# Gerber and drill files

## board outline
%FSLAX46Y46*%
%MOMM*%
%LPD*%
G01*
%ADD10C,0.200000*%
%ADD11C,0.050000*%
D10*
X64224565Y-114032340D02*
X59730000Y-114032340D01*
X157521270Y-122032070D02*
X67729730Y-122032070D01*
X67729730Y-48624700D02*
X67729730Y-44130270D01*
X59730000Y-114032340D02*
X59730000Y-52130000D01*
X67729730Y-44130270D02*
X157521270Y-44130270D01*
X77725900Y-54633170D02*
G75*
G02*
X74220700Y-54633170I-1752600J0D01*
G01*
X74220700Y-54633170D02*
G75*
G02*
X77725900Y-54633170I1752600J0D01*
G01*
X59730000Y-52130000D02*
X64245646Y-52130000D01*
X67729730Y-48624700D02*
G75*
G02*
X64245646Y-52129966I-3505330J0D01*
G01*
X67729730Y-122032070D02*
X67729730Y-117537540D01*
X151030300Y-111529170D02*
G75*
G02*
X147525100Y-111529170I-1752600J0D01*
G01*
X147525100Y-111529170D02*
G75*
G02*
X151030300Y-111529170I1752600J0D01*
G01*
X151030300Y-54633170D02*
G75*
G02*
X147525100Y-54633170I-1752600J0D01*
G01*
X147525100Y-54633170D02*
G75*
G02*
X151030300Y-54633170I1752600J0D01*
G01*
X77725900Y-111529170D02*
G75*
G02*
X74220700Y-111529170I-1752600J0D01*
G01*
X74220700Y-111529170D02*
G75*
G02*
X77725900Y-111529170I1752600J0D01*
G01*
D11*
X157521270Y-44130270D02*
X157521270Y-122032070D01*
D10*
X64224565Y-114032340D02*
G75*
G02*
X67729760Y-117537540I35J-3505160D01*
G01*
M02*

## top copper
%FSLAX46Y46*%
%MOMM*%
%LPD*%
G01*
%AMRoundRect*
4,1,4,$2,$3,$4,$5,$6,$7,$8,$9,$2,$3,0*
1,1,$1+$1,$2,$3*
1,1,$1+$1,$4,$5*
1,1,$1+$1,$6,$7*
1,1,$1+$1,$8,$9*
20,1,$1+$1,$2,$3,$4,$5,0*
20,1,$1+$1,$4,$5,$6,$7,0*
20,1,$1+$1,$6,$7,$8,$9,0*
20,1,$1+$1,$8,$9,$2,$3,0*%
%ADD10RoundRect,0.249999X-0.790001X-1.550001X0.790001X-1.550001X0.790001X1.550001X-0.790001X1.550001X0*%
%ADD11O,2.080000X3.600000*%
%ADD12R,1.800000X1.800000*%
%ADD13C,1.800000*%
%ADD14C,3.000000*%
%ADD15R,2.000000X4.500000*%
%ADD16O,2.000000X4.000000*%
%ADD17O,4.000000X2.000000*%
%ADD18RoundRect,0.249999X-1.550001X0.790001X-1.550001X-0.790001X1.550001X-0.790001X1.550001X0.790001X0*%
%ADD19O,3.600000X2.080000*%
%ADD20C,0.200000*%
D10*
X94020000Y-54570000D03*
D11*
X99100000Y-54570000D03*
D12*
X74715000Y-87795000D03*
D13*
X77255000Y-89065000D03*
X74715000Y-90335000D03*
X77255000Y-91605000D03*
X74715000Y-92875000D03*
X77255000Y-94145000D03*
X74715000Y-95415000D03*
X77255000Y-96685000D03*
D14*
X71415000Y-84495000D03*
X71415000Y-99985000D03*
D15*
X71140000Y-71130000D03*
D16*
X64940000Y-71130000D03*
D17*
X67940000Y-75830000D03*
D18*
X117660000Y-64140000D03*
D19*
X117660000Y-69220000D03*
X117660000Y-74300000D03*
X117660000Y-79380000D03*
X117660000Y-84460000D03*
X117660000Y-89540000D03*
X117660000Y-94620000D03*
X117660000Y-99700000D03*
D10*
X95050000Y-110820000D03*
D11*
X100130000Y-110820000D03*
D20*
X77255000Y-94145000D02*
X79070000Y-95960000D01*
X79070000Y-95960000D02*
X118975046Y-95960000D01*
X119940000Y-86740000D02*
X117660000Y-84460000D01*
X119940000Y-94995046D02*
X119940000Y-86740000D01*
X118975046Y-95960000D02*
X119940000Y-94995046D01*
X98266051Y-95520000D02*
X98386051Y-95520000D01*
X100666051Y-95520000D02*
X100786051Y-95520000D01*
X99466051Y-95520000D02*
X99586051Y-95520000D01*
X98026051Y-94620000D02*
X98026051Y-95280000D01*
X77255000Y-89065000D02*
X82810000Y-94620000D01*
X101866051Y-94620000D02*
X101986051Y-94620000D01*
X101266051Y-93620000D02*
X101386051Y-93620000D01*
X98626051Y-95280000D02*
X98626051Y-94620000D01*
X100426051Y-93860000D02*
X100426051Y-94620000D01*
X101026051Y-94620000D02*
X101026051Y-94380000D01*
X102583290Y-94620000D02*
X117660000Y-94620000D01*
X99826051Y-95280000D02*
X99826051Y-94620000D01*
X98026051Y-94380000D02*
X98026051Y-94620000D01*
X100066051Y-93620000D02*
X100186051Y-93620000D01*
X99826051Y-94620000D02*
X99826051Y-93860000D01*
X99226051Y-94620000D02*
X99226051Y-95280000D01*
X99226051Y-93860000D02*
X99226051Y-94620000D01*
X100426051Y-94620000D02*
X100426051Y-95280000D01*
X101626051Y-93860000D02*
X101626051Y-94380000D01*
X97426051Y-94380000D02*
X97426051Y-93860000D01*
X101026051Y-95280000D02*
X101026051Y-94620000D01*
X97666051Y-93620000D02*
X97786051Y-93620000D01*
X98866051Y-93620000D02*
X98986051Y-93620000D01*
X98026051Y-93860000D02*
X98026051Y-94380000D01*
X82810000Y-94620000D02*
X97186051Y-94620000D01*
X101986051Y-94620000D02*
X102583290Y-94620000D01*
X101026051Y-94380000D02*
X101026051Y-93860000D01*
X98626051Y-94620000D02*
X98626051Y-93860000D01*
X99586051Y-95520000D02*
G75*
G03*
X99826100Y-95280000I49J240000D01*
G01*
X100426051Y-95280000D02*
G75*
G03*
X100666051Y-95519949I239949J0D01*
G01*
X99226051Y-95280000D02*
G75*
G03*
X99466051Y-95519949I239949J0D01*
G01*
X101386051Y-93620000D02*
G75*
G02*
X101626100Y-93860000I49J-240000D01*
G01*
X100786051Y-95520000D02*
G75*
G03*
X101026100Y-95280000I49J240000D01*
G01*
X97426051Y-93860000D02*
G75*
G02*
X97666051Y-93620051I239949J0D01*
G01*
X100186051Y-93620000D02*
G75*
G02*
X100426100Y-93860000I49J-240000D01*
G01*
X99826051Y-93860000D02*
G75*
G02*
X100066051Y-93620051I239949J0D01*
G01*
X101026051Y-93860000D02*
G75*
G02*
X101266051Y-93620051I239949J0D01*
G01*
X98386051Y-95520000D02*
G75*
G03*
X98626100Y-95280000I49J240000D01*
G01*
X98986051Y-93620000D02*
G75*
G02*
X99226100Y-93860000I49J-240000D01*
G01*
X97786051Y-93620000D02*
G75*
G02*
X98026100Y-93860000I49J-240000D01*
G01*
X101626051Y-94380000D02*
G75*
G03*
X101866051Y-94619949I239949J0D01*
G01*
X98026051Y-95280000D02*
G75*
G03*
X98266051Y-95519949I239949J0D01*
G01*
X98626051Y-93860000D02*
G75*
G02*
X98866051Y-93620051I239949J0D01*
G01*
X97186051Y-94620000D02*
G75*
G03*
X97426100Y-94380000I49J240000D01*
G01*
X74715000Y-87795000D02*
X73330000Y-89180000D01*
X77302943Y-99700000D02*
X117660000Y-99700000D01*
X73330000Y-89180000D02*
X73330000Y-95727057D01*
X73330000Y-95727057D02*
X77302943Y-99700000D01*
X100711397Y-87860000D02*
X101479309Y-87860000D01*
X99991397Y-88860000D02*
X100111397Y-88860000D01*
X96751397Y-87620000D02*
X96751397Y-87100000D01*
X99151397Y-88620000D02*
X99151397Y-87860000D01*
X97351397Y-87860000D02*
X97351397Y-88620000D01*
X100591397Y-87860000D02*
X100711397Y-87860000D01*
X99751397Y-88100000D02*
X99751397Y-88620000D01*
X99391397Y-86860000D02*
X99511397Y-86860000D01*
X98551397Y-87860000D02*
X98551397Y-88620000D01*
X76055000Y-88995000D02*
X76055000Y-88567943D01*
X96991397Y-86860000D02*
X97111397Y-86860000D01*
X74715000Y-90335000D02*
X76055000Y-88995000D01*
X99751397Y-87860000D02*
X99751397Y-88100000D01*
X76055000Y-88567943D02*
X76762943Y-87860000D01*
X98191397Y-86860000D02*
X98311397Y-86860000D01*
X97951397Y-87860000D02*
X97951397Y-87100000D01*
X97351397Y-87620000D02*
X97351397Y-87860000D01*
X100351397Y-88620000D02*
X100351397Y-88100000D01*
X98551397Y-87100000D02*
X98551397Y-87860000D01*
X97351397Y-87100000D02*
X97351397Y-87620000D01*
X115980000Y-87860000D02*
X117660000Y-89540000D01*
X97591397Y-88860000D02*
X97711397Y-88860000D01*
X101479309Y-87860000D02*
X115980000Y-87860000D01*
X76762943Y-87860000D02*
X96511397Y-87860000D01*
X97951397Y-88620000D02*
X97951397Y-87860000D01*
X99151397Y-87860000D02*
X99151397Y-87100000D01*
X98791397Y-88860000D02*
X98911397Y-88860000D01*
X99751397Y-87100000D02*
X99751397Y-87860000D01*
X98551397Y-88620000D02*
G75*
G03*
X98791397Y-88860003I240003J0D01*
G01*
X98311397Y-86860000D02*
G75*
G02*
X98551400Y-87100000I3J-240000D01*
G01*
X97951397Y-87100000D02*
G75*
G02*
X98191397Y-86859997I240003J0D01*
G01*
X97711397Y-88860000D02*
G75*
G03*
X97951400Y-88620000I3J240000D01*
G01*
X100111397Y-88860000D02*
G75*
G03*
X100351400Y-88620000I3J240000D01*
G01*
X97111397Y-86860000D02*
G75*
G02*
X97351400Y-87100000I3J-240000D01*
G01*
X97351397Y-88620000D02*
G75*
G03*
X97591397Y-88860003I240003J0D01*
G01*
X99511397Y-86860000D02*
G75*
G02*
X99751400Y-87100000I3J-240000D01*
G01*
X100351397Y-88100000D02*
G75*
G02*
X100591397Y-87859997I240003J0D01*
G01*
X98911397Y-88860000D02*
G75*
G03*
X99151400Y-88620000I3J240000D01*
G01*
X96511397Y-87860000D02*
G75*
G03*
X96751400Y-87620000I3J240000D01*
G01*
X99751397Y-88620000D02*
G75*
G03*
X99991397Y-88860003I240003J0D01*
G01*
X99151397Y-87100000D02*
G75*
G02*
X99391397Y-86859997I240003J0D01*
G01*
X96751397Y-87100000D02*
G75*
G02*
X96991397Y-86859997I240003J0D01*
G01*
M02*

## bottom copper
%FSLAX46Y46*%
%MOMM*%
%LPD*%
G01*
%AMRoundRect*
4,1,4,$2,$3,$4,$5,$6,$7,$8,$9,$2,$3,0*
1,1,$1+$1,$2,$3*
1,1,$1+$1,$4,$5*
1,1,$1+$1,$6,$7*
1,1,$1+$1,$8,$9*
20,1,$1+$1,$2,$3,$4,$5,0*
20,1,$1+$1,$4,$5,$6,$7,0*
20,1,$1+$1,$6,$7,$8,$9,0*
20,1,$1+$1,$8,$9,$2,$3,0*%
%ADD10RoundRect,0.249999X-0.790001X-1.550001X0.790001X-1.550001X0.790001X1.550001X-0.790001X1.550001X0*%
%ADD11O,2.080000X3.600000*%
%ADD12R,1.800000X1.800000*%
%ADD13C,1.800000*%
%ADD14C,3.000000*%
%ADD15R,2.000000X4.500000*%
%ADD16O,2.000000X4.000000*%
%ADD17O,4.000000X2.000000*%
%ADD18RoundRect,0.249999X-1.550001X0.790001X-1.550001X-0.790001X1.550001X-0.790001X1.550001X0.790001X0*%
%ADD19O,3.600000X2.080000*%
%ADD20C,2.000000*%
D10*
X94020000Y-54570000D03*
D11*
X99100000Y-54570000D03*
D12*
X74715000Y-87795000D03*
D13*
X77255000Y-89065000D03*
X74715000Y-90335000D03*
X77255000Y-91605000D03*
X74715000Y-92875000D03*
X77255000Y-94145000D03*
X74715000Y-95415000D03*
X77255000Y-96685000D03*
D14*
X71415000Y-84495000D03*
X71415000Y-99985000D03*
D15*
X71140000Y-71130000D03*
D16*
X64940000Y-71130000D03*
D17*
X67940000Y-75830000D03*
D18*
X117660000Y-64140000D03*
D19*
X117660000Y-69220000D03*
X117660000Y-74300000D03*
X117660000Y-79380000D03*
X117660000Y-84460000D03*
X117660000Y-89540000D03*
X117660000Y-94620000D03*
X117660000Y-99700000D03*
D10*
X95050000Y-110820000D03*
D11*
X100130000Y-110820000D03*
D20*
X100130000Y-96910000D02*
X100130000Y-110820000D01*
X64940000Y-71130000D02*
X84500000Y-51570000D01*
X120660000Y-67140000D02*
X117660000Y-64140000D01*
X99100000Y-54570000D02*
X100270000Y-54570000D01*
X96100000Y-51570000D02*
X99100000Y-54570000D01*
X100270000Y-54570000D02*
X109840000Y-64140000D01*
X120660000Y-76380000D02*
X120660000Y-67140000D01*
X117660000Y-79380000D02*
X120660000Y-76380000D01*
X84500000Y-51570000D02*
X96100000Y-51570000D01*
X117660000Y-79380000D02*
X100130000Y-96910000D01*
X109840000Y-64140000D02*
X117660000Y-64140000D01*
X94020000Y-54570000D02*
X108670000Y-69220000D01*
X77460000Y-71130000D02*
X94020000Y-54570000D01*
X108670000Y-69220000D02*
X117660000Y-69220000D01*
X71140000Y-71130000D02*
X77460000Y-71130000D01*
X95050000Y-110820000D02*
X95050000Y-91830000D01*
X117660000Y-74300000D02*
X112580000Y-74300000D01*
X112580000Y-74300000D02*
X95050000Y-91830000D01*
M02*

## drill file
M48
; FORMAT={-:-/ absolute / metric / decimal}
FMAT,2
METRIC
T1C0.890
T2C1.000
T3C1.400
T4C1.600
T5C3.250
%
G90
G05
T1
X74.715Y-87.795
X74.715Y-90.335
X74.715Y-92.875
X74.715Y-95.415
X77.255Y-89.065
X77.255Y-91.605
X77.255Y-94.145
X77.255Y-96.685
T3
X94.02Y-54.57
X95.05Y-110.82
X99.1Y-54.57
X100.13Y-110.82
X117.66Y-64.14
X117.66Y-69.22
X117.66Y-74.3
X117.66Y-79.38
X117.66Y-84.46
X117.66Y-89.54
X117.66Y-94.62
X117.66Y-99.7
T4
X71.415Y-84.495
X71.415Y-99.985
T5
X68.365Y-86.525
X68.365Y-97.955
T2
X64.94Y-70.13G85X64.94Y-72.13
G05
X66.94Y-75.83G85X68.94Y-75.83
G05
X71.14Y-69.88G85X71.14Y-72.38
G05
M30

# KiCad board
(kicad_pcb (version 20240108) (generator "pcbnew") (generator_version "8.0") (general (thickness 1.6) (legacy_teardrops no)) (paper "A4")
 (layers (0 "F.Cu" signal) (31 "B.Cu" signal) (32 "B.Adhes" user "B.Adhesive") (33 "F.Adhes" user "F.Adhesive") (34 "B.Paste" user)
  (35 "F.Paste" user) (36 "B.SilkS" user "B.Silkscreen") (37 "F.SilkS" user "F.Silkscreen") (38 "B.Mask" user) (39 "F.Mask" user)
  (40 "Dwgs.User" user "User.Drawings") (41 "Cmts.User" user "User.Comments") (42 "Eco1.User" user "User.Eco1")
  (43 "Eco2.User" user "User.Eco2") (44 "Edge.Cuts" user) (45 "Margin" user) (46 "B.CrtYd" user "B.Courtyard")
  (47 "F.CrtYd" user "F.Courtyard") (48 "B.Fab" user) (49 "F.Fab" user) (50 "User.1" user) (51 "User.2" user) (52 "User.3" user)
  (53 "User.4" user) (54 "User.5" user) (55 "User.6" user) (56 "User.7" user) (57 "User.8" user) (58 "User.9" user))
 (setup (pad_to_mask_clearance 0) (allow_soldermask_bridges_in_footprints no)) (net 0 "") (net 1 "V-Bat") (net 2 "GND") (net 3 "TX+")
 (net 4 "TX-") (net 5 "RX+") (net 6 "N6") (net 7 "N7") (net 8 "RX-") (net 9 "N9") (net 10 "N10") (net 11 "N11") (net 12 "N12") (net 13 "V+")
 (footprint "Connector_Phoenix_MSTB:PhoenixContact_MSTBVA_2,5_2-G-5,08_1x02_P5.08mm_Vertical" (layer "F.Cu") (at 94.02 54.57)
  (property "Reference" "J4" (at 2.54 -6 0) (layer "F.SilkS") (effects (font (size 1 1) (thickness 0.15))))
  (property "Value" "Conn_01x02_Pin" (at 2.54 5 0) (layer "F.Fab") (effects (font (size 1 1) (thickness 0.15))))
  (pad "1" thru_hole roundrect (at 0 0) (size 2.08 3.6) (drill 1.4) (layers "*.Cu" "*.Mask") (remove_unused_layers no)
   (roundrect_rratio 0.120192) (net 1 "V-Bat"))
  (pad "2" thru_hole oval (at 5.08 0) (size 2.08 3.6) (drill 1.4) (layers "*.Cu" "*.Mask") (remove_unused_layers no) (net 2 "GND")))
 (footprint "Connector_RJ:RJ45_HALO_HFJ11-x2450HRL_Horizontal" (layer "F.Cu") (at 74.715 87.795 -90)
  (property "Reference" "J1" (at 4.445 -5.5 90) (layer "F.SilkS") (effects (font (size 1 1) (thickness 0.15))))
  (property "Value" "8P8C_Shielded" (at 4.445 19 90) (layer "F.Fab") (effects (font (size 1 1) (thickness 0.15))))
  (pad "" np_thru_hole circle (at -1.27 6.35 270) (size 3.25 3.25) (drill 3.25) (layers "*.Cu" "*.Mask"))
  (pad "" np_thru_hole circle (at 10.16 6.35 270) (size 3.25 3.25) (drill 3.25) (layers "*.Cu" "*.Mask"))
  (pad "1" thru_hole rect (at 0 0 270) (size 1.8 1.8) (drill 0.89) (layers "*.Cu" "*.Mask") (remove_unused_layers no) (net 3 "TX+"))
  (pad "2" thru_hole circle (at 1.27 -2.54 270) (size 1.8 1.8) (drill 0.89) (layers "*.Cu" "*.Mask") (remove_unused_layers no) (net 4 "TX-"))
  (pad "3" thru_hole circle (at 2.54 0 270) (size 1.8 1.8) (drill 0.89) (layers "*.Cu" "*.Mask") (remove_unused_layers no) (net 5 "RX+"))
  (pad "4" thru_hole circle (at 3.81 -2.54 270) (size 1.8 1.8) (drill 0.89) (layers "*.Cu" "*.Mask") (remove_unused_layers no) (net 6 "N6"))
  (pad "5" thru_hole circle (at 5.08 0 270) (size 1.8 1.8) (drill 0.89) (layers "*.Cu" "*.Mask") (remove_unused_layers no) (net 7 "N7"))
  (pad "6" thru_hole circle (at 6.35 -2.54 270) (size 1.8 1.8) (drill 0.89) (layers "*.Cu" "*.Mask") (remove_unused_layers no) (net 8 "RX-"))
  (pad "7" thru_hole circle (at 7.62 0 270) (size 1.8 1.8) (drill 0.89) (layers "*.Cu" "*.Mask") (remove_unused_layers no) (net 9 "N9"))
  (pad "8" thru_hole circle (at 8.89 -2.54 270) (size 1.8 1.8) (drill 0.89) (layers "*.Cu" "*.Mask") (remove_unused_layers no)
   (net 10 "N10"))
  (pad "SH" thru_hole circle (at -3.3 3.3 270) (size 3 3) (drill 1.6) (layers "*.Cu" "*.Mask") (remove_unused_layers no) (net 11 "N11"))
  (pad "SH" thru_hole circle (at 12.19 3.3 270) (size 3 3) (drill 1.6) (layers "*.Cu" "*.Mask") (remove_unused_layers no) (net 11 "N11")))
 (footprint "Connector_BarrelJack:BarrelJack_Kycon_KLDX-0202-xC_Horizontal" (layer "F.Cu") (at 71.14 71.13)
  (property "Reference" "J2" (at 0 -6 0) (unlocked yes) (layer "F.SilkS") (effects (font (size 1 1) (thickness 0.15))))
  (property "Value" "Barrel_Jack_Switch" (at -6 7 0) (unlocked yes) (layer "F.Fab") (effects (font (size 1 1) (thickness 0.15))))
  (pad "1" thru_hole rect (at 0 0) (size 2 4.5) (drill oval 1 3.5) (layers "*.Cu" "*.Mask") (remove_unused_layers no) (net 1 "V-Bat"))
  (pad "2" thru_hole oval (at -6.2 0) (size 2 4) (drill oval 1 3) (layers "*.Cu" "*.Mask") (remove_unused_layers no) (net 2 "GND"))
  (pad "3" thru_hole oval (at -3.2 4.7 90) (size 2 4) (drill oval 1 3) (layers "*.Cu" "*.Mask") (remove_unused_layers no) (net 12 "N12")))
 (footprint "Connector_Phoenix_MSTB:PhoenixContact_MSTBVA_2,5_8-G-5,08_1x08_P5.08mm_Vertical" (layer "F.Cu") (at 117.66 64.14 -90)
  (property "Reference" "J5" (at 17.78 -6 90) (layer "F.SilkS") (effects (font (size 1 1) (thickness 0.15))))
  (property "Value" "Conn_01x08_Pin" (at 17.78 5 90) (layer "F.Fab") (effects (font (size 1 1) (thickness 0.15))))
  (pad "1" thru_hole roundrect (at 0 0 270) (size 2.08 3.6) (drill 1.4) (layers "*.Cu" "*.Mask") (remove_unused_layers no)
   (roundrect_rratio 0.120192) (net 2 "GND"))
  (pad "2" thru_hole oval (at 5.08 0 270) (size 2.08 3.6) (drill 1.4) (layers "*.Cu" "*.Mask") (remove_unused_layers no) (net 1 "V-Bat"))
  (pad "3" thru_hole oval (at 10.16 0 270) (size 2.08 3.6) (drill 1.4) (layers "*.Cu" "*.Mask") (remove_unused_layers no) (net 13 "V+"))
  (pad "4" thru_hole oval (at 15.24 0 270) (size 2.08 3.6) (drill 1.4) (layers "*.Cu" "*.Mask") (remove_unused_layers no) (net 2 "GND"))
  (pad "5" thru_hole oval (at 20.32 0 270) (size 2.08 3.6) (drill 1.4) (layers "*.Cu" "*.Mask") (remove_unused_layers no) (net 8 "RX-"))
  (pad "6" thru_hole oval (at 25.4 0 270) (size 2.08 3.6) (drill 1.4) (layers "*.Cu" "*.Mask") (remove_unused_layers no) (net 5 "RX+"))
  (pad "7" thru_hole oval (at 30.48 0 270) (size 2.08 3.6) (drill 1.4) (layers "*.Cu" "*.Mask") (remove_unused_layers no) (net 4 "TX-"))
  (pad "8" thru_hole oval (at 35.56 0 270) (size 2.08 3.6) (drill 1.4) (layers "*.Cu" "*.Mask") (remove_unused_layers no) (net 3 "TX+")))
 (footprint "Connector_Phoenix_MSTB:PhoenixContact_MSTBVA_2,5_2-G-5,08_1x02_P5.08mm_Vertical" (layer "F.Cu") (at 95.05 110.82)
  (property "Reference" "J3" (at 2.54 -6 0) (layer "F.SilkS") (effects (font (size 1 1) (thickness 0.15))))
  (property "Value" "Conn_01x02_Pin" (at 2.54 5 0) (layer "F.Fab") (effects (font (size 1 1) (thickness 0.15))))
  (pad "1" thru_hole roundrect (at 0 0) (size 2.08 3.6) (drill 1.4) (layers "*.Cu" "*.Mask") (remove_unused_layers no)
   (roundrect_rratio 0.120192) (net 13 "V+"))
  (pad "2" thru_hole oval (at 5.08 0) (size 2.08 3.6) (drill 1.4) (layers "*.Cu" "*.Mask") (remove_unused_layers no) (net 2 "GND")))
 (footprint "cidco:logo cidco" (layer "F.Cu") (at 94.433078 70.444943)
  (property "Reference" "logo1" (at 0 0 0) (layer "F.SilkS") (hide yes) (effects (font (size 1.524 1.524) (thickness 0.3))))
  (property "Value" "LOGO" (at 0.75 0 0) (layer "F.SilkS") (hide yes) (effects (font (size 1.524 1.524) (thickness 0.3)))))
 (gr_line (start 64.224565 114.03234) (end 59.73 114.03234) (stroke (width 0.2) (type default)) (layer "Edge.Cuts"))
 (gr_line (start 157.52127 122.03207) (end 67.72973 122.03207) (stroke (width 0.2) (type default)) (layer "Edge.Cuts"))
 (gr_line (start 67.72973 48.6247) (end 67.72973 44.13027) (stroke (width 0.2) (type default)) (layer "Edge.Cuts"))
 (gr_line (start 59.73 114.03234) (end 59.73 52.13) (stroke (width 0.2) (type default)) (layer "Edge.Cuts"))
 (gr_line (start 67.72973 44.13027) (end 157.52127 44.13027) (stroke (width 0.2) (type default)) (layer "Edge.Cuts"))
 (gr_circle (center 75.9733 54.63317) (end 77.7259 54.63317) (stroke (width 0.2) (type default)) (fill none) (layer "Edge.Cuts"))
 (gr_line (start 59.73 52.13) (end 64.245646 52.13) (stroke (width 0.2) (type default)) (layer "Edge.Cuts"))
 (gr_arc (start 67.72973 48.6247) (mid 66.710545 51.095832) (end 64.245646 52.13) (stroke (width 0.2) (type default)) (layer "Edge.Cuts"))
 (gr_line (start 67.72973 122.03207) (end 67.72973 117.53754) (stroke (width 0.2) (type default)) (layer "Edge.Cuts"))
 (gr_circle (center 149.2777 111.52917) (end 151.0303 111.52917) (stroke (width 0.2) (type default)) (fill none) (layer "Edge.Cuts"))
 (gr_circle (center 149.2777 54.63317) (end 151.0303 54.63317) (stroke (width 0.2) (type default)) (fill none) (layer "Edge.Cuts"))
 (gr_circle (center 75.9733 111.52917) (end 77.7259 111.52917) (stroke (width 0.2) (type default)) (fill none) (layer "Edge.Cuts"))
 (gr_line (start 157.52127 44.13027) (end 157.52127 122.03207) (stroke (width 0.05) (type default)) (layer "Edge.Cuts"))
 (gr_arc (start 64.224565 114.03234) (mid 66.703102 115.058992) (end 67.72973 117.53754) (stroke (width 0.2) (type default))
  (layer "Edge.Cuts"))
 (segment (start 77.255 94.145) (end 79.07 95.96) (width 0.2) (layer "F.Cu") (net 8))
 (segment (start 79.07 95.96) (end 118.975046 95.96) (width 0.2) (layer "F.Cu") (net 8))
 (segment (start 119.94 86.74) (end 117.66 84.46) (width 0.2) (layer "F.Cu") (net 8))
 (segment (start 119.94 94.995046) (end 119.94 86.74) (width 0.2) (layer "F.Cu") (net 8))
 (segment (start 118.975046 95.96) (end 119.94 94.995046) (width 0.2) (layer "F.Cu") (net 8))
 (segment (start 98.266051 95.52) (end 98.386051 95.52) (width 0.2) (layer "F.Cu") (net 4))
 (segment (start 100.666051 95.52) (end 100.786051 95.52) (width 0.2) (layer "F.Cu") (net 4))
 (segment (start 99.466051 95.52) (end 99.586051 95.52) (width 0.2) (layer "F.Cu") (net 4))
 (segment (start 98.026051 94.62) (end 98.026051 95.28) (width 0.2) (layer "F.Cu") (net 4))
 (segment (start 77.255 89.065) (end 82.81 94.62) (width 0.2) (layer "F.Cu") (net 4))
 (segment (start 101.866051 94.62) (end 101.986051 94.62) (width 0.2) (layer "F.Cu") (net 4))
 (segment (start 101.266051 93.62) (end 101.386051 93.62) (width 0.2) (layer "F.Cu") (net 4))
 (segment (start 98.626051 95.28) (end 98.626051 94.62) (width 0.2) (layer "F.Cu") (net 4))
 (segment (start 100.426051 93.86) (end 100.426051 94.62) (width 0.2) (layer "F.Cu") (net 4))
 (segment (start 101.026051 94.62) (end 101.026051 94.38) (width 0.2) (layer "F.Cu") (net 4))
 (segment (start 102.58329 94.62) (end 117.66 94.62) (width 0.2) (layer "F.Cu") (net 4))
 (segment (start 99.826051 95.28) (end 99.826051 94.62) (width 0.2) (layer "F.Cu") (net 4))
 (segment (start 98.026051 94.38) (end 98.026051 94.62) (width 0.2) (layer "F.Cu") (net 4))
 (segment (start 100.066051 93.62) (end 100.186051 93.62) (width 0.2) (layer "F.Cu") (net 4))
 (segment (start 99.826051 94.62) (end 99.826051 93.86) (width 0.2) (layer "F.Cu") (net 4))
 (segment (start 99.226051 94.62) (end 99.226051 95.28) (width 0.2) (layer "F.Cu") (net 4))
 (segment (start 99.226051 93.86) (end 99.226051 94.62) (width 0.2) (layer "F.Cu") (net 4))
 (segment (start 100.426051 94.62) (end 100.426051 95.28) (width 0.2) (layer "F.Cu") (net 4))
 (segment (start 101.626051 93.86) (end 101.626051 94.38) (width 0.2) (layer "F.Cu") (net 4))
 (segment (start 97.426051 94.38) (end 97.426051 93.86) (width 0.2) (layer "F.Cu") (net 4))
 (segment (start 101.026051 95.28) (end 101.026051 94.62) (width 0.2) (layer "F.Cu") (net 4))
 (segment (start 97.666051 93.62) (end 97.786051 93.62) (width 0.2) (layer "F.Cu") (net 4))
 (segment (start 98.866051 93.62) (end 98.986051 93.62) (width 0.2) (layer "F.Cu") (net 4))
 (segment (start 98.026051 93.86) (end 98.026051 94.38) (width 0.2) (layer "F.Cu") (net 4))
 (segment (start 82.81 94.62) (end 97.186051 94.62) (width 0.2) (layer "F.Cu") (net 4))
 (segment (start 101.986051 94.62) (end 102.58329 94.62) (width 0.2) (layer "F.Cu") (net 4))
 (segment (start 101.026051 94.38) (end 101.026051 93.86) (width 0.2) (layer "F.Cu") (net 4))
 (segment (start 98.626051 94.62) (end 98.626051 93.86) (width 0.2) (layer "F.Cu") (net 4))
 (arc (start 99.586051 95.52) (mid 99.755757 95.449706) (end 99.826051 95.28) (width 0.2) (layer "F.Cu") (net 4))
 (arc (start 100.426051 95.28) (mid 100.496345 95.449706) (end 100.666051 95.52) (width 0.2) (layer "F.Cu") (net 4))
 (arc (start 99.226051 95.28) (mid 99.296345 95.449706) (end 99.466051 95.52) (width 0.2) (layer "F.Cu") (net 4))
 (arc (start 101.386051 93.62) (mid 101.555757 93.690294) (end 101.626051 93.86) (width 0.2) (layer "F.Cu") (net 4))
 (arc (start 100.786051 95.52) (mid 100.955757 95.449706) (end 101.026051 95.28) (width 0.2) (layer "F.Cu") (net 4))
 (arc (start 97.426051 93.86) (mid 97.496345 93.690294) (end 97.666051 93.62) (width 0.2) (layer "F.Cu") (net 4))
 (arc (start 100.186051 93.62) (mid 100.355757 93.690294) (end 100.426051 93.86) (width 0.2) (layer "F.Cu") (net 4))
 (arc (start 99.826051 93.86) (mid 99.896345 93.690294) (end 100.066051 93.62) (width 0.2) (layer "F.Cu") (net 4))
 (arc (start 101.026051 93.86) (mid 101.096345 93.690294) (end 101.266051 93.62) (width 0.2) (layer "F.Cu") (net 4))
 (arc (start 98.386051 95.52) (mid 98.555757 95.449706) (end 98.626051 95.28) (width 0.2) (layer "F.Cu") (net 4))
 (arc (start 98.986051 93.62) (mid 99.155757 93.690294) (end 99.226051 93.86) (width 0.2) (layer "F.Cu") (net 4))
 (arc (start 97.786051 93.62) (mid 97.955757 93.690294) (end 98.026051 93.86) (width 0.2) (layer "F.Cu") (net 4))
 (arc (start 101.626051 94.38) (mid 101.696345 94.549706) (end 101.866051 94.62) (width 0.2) (layer "F.Cu") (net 4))
 (arc (start 98.026051 95.28) (mid 98.096345 95.449706) (end 98.266051 95.52) (width 0.2) (layer "F.Cu") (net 4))
 (arc (start 98.626051 93.86) (mid 98.696345 93.690294) (end 98.866051 93.62) (width 0.2) (layer "F.Cu") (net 4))
 (arc (start 97.186051 94.62) (mid 97.355757 94.549706) (end 97.426051 94.38) (width 0.2) (layer "F.Cu") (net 4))
 (segment (start 74.715 87.795) (end 73.33 89.18) (width 0.2) (layer "F.Cu") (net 3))
 (segment (start 77.302943 99.7) (end 117.66 99.7) (width 0.2) (layer "F.Cu") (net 3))
 (segment (start 73.33 89.18) (end 73.33 95.727057) (width 0.2) (layer "F.Cu") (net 3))
 (segment (start 73.33 95.727057) (end 77.302943 99.7) (width 0.2) (layer "F.Cu") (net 3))
 (segment (start 100.711397 87.86) (end 101.479309 87.86) (width 0.2) (layer "F.Cu") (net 5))
 (segment (start 99.991397 88.86) (end 100.111397 88.86) (width 0.2) (layer "F.Cu") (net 5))
 (segment (start 96.751397 87.62) (end 96.751397 87.1) (width 0.2) (layer "F.Cu") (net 5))
 (segment (start 99.151397 88.62) (end 99.151397 87.86) (width 0.2) (layer "F.Cu") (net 5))
 (segment (start 97.351397 87.86) (end 97.351397 88.62) (width 0.2) (layer "F.Cu") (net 5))
 (segment (start 100.591397 87.86) (end 100.711397 87.86) (width 0.2) (layer "F.Cu") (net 5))
 (segment (start 99.751397 88.1) (end 99.751397 88.62) (width 0.2) (layer "F.Cu") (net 5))
 (segment (start 99.391397 86.86) (end 99.511397 86.86) (width 0.2) (layer "F.Cu") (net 5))
 (segment (start 98.551397 87.86) (end 98.551397 88.62) (width 0.2) (layer "F.Cu") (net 5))
 (segment (start 76.055 88.995) (end 76.055 88.567943) (width 0.2) (layer "F.Cu") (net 5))
 (segment (start 96.991397 86.86) (end 97.111397 86.86) (width 0.2) (layer "F.Cu") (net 5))
 (segment (start 74.715 90.335) (end 76.055 88.995) (width 0.2) (layer "F.Cu") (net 5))
 (segment (start 99.751397 87.86) (end 99.751397 88.1) (width 0.2) (layer "F.Cu") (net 5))
 (segment (start 76.055 88.567943) (end 76.762943 87.86) (width 0.2) (layer "F.Cu") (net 5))
 (segment (start 98.191397 86.86) (end 98.311397 86.86) (width 0.2) (layer "F.Cu") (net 5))
 (segment (start 97.951397 87.86) (end 97.951397 87.1) (width 0.2) (layer "F.Cu") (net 5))
 (segment (start 97.351397 87.62) (end 97.351397 87.86) (width 0.2) (layer "F.Cu") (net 5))
 (segment (start 100.351397 88.62) (end 100.351397 88.1) (width 0.2) (layer "F.Cu") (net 5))
 (segment (start 98.551397 87.1) (end 98.551397 87.86) (width 0.2) (layer "F.Cu") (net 5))
 (segment (start 97.351397 87.1) (end 97.351397 87.62) (width 0.2) (layer "F.Cu") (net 5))
 (segment (start 115.98 87.86) (end 117.66 89.54) (width 0.2) (layer "F.Cu") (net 5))
 (segment (start 97.591397 88.86) (end 97.711397 88.86) (width 0.2) (layer "F.Cu") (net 5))
 (segment (start 101.479309 87.86) (end 115.98 87.86) (width 0.2) (layer "F.Cu") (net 5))
 (segment (start 76.762943 87.86) (end 96.511397 87.86) (width 0.2) (layer "F.Cu") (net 5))
 (segment (start 97.951397 88.62) (end 97.951397 87.86) (width 0.2) (layer "F.Cu") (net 5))
 (segment (start 99.151397 87.86) (end 99.151397 87.1) (width 0.2) (layer "F.Cu") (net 5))
 (segment (start 98.791397 88.86) (end 98.911397 88.86) (width 0.2) (layer "F.Cu") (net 5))
 (segment (start 99.751397 87.1) (end 99.751397 87.86) (width 0.2) (layer "F.Cu") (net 5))
 (arc (start 98.551397 88.62) (mid 98.621691 88.789706) (end 98.791397 88.86) (width 0.2) (layer "F.Cu") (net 5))
 (arc (start 98.311397 86.86) (mid 98.481103 86.930294) (end 98.551397 87.1) (width 0.2) (layer "F.Cu") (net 5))
 (arc (start 97.951397 87.1) (mid 98.021691 86.930294) (end 98.191397 86.86) (width 0.2) (layer "F.Cu") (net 5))
 (arc (start 97.711397 88.86) (mid 97.881103 88.789706) (end 97.951397 88.62) (width 0.2) (layer "F.Cu") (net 5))
 (arc (start 100.111397 88.86) (mid 100.281103 88.789706) (end 100.351397 88.62) (width 0.2) (layer "F.Cu") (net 5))
 (arc (start 97.111397 86.86) (mid 97.281103 86.930294) (end 97.351397 87.1) (width 0.2) (layer "F.Cu") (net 5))
 (arc (start 97.351397 88.62) (mid 97.421691 88.789706) (end 97.591397 88.86) (width 0.2) (layer "F.Cu") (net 5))
 (arc (start 99.511397 86.86) (mid 99.681103 86.930294) (end 99.751397 87.1) (width 0.2) (layer "F.Cu") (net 5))
 (arc (start 100.351397 88.1) (mid 100.421691 87.930294) (end 100.591397 87.86) (width 0.2) (layer "F.Cu") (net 5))
 (arc (start 98.911397 88.86) (mid 99.081103 88.789706) (end 99.151397 88.62) (width 0.2) (layer "F.Cu") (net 5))
 (arc (start 96.511397 87.86) (mid 96.681103 87.789706) (end 96.751397 87.62) (width 0.2) (layer "F.Cu") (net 5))
 (arc (start 99.751397 88.62) (mid 99.821691 88.789706) (end 99.991397 88.86) (width 0.2) (layer "F.Cu") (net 5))
 (arc (start 99.151397 87.1) (mid 99.221691 86.930294) (end 99.391397 86.86) (width 0.2) (layer "F.Cu") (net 5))
 (arc (start 96.751397 87.1) (mid 96.821691 86.930294) (end 96.991397 86.86) (width 0.2) (layer "F.Cu") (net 5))
 (segment (start 100.13 96.91) (end 100.13 110.82) (width 2) (layer "B.Cu") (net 2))
 (segment (start 64.94 71.13) (end 84.5 51.57) (width 2) (layer "B.Cu") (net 2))
 (segment (start 120.66 67.14) (end 117.66 64.14) (width 2) (layer "B.Cu") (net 2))
 (segment (start 99.1 54.57) (end 100.27 54.57) (width 2) (layer "B.Cu") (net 2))
 (segment (start 96.1 51.57) (end 99.1 54.57) (width 2) (layer "B.Cu") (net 2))
 (segment (start 100.27 54.57) (end 109.84 64.14) (width 2) (layer "B.Cu") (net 2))
 (segment (start 120.66 76.38) (end 120.66 67.14) (width 2) (layer "B.Cu") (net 2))
 (segment (start 117.66 79.38) (end 120.66 76.38) (width 2) (layer "B.Cu") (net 2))
 (segment (start 84.5 51.57) (end 96.1 51.57) (width 2) (layer "B.Cu") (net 2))
 (segment (start 117.66 79.38) (end 100.13 96.91) (width 2) (layer "B.Cu") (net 2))
 (segment (start 109.84 64.14) (end 117.66 64.14) (width 2) (layer "B.Cu") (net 2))
 (segment (start 94.02 54.57) (end 108.67 69.22) (width 2) (layer "B.Cu") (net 1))
 (segment (start 77.46 71.13) (end 94.02 54.57) (width 2) (layer "B.Cu") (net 1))
 (segment (start 108.67 69.22) (end 117.66 69.22) (width 2) (layer "B.Cu") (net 1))
 (segment (start 71.14 71.13) (end 77.46 71.13) (width 2) (layer "B.Cu") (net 1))
 (segment (start 95.05 110.82) (end 95.05 91.83) (width 2) (layer "B.Cu") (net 13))
 (segment (start 117.66 74.3) (end 112.58 74.3) (width 2) (layer "B.Cu") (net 13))
 (segment (start 112.58 74.3) (end 95.05 91.83) (width 2) (layer "B.Cu") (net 13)))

